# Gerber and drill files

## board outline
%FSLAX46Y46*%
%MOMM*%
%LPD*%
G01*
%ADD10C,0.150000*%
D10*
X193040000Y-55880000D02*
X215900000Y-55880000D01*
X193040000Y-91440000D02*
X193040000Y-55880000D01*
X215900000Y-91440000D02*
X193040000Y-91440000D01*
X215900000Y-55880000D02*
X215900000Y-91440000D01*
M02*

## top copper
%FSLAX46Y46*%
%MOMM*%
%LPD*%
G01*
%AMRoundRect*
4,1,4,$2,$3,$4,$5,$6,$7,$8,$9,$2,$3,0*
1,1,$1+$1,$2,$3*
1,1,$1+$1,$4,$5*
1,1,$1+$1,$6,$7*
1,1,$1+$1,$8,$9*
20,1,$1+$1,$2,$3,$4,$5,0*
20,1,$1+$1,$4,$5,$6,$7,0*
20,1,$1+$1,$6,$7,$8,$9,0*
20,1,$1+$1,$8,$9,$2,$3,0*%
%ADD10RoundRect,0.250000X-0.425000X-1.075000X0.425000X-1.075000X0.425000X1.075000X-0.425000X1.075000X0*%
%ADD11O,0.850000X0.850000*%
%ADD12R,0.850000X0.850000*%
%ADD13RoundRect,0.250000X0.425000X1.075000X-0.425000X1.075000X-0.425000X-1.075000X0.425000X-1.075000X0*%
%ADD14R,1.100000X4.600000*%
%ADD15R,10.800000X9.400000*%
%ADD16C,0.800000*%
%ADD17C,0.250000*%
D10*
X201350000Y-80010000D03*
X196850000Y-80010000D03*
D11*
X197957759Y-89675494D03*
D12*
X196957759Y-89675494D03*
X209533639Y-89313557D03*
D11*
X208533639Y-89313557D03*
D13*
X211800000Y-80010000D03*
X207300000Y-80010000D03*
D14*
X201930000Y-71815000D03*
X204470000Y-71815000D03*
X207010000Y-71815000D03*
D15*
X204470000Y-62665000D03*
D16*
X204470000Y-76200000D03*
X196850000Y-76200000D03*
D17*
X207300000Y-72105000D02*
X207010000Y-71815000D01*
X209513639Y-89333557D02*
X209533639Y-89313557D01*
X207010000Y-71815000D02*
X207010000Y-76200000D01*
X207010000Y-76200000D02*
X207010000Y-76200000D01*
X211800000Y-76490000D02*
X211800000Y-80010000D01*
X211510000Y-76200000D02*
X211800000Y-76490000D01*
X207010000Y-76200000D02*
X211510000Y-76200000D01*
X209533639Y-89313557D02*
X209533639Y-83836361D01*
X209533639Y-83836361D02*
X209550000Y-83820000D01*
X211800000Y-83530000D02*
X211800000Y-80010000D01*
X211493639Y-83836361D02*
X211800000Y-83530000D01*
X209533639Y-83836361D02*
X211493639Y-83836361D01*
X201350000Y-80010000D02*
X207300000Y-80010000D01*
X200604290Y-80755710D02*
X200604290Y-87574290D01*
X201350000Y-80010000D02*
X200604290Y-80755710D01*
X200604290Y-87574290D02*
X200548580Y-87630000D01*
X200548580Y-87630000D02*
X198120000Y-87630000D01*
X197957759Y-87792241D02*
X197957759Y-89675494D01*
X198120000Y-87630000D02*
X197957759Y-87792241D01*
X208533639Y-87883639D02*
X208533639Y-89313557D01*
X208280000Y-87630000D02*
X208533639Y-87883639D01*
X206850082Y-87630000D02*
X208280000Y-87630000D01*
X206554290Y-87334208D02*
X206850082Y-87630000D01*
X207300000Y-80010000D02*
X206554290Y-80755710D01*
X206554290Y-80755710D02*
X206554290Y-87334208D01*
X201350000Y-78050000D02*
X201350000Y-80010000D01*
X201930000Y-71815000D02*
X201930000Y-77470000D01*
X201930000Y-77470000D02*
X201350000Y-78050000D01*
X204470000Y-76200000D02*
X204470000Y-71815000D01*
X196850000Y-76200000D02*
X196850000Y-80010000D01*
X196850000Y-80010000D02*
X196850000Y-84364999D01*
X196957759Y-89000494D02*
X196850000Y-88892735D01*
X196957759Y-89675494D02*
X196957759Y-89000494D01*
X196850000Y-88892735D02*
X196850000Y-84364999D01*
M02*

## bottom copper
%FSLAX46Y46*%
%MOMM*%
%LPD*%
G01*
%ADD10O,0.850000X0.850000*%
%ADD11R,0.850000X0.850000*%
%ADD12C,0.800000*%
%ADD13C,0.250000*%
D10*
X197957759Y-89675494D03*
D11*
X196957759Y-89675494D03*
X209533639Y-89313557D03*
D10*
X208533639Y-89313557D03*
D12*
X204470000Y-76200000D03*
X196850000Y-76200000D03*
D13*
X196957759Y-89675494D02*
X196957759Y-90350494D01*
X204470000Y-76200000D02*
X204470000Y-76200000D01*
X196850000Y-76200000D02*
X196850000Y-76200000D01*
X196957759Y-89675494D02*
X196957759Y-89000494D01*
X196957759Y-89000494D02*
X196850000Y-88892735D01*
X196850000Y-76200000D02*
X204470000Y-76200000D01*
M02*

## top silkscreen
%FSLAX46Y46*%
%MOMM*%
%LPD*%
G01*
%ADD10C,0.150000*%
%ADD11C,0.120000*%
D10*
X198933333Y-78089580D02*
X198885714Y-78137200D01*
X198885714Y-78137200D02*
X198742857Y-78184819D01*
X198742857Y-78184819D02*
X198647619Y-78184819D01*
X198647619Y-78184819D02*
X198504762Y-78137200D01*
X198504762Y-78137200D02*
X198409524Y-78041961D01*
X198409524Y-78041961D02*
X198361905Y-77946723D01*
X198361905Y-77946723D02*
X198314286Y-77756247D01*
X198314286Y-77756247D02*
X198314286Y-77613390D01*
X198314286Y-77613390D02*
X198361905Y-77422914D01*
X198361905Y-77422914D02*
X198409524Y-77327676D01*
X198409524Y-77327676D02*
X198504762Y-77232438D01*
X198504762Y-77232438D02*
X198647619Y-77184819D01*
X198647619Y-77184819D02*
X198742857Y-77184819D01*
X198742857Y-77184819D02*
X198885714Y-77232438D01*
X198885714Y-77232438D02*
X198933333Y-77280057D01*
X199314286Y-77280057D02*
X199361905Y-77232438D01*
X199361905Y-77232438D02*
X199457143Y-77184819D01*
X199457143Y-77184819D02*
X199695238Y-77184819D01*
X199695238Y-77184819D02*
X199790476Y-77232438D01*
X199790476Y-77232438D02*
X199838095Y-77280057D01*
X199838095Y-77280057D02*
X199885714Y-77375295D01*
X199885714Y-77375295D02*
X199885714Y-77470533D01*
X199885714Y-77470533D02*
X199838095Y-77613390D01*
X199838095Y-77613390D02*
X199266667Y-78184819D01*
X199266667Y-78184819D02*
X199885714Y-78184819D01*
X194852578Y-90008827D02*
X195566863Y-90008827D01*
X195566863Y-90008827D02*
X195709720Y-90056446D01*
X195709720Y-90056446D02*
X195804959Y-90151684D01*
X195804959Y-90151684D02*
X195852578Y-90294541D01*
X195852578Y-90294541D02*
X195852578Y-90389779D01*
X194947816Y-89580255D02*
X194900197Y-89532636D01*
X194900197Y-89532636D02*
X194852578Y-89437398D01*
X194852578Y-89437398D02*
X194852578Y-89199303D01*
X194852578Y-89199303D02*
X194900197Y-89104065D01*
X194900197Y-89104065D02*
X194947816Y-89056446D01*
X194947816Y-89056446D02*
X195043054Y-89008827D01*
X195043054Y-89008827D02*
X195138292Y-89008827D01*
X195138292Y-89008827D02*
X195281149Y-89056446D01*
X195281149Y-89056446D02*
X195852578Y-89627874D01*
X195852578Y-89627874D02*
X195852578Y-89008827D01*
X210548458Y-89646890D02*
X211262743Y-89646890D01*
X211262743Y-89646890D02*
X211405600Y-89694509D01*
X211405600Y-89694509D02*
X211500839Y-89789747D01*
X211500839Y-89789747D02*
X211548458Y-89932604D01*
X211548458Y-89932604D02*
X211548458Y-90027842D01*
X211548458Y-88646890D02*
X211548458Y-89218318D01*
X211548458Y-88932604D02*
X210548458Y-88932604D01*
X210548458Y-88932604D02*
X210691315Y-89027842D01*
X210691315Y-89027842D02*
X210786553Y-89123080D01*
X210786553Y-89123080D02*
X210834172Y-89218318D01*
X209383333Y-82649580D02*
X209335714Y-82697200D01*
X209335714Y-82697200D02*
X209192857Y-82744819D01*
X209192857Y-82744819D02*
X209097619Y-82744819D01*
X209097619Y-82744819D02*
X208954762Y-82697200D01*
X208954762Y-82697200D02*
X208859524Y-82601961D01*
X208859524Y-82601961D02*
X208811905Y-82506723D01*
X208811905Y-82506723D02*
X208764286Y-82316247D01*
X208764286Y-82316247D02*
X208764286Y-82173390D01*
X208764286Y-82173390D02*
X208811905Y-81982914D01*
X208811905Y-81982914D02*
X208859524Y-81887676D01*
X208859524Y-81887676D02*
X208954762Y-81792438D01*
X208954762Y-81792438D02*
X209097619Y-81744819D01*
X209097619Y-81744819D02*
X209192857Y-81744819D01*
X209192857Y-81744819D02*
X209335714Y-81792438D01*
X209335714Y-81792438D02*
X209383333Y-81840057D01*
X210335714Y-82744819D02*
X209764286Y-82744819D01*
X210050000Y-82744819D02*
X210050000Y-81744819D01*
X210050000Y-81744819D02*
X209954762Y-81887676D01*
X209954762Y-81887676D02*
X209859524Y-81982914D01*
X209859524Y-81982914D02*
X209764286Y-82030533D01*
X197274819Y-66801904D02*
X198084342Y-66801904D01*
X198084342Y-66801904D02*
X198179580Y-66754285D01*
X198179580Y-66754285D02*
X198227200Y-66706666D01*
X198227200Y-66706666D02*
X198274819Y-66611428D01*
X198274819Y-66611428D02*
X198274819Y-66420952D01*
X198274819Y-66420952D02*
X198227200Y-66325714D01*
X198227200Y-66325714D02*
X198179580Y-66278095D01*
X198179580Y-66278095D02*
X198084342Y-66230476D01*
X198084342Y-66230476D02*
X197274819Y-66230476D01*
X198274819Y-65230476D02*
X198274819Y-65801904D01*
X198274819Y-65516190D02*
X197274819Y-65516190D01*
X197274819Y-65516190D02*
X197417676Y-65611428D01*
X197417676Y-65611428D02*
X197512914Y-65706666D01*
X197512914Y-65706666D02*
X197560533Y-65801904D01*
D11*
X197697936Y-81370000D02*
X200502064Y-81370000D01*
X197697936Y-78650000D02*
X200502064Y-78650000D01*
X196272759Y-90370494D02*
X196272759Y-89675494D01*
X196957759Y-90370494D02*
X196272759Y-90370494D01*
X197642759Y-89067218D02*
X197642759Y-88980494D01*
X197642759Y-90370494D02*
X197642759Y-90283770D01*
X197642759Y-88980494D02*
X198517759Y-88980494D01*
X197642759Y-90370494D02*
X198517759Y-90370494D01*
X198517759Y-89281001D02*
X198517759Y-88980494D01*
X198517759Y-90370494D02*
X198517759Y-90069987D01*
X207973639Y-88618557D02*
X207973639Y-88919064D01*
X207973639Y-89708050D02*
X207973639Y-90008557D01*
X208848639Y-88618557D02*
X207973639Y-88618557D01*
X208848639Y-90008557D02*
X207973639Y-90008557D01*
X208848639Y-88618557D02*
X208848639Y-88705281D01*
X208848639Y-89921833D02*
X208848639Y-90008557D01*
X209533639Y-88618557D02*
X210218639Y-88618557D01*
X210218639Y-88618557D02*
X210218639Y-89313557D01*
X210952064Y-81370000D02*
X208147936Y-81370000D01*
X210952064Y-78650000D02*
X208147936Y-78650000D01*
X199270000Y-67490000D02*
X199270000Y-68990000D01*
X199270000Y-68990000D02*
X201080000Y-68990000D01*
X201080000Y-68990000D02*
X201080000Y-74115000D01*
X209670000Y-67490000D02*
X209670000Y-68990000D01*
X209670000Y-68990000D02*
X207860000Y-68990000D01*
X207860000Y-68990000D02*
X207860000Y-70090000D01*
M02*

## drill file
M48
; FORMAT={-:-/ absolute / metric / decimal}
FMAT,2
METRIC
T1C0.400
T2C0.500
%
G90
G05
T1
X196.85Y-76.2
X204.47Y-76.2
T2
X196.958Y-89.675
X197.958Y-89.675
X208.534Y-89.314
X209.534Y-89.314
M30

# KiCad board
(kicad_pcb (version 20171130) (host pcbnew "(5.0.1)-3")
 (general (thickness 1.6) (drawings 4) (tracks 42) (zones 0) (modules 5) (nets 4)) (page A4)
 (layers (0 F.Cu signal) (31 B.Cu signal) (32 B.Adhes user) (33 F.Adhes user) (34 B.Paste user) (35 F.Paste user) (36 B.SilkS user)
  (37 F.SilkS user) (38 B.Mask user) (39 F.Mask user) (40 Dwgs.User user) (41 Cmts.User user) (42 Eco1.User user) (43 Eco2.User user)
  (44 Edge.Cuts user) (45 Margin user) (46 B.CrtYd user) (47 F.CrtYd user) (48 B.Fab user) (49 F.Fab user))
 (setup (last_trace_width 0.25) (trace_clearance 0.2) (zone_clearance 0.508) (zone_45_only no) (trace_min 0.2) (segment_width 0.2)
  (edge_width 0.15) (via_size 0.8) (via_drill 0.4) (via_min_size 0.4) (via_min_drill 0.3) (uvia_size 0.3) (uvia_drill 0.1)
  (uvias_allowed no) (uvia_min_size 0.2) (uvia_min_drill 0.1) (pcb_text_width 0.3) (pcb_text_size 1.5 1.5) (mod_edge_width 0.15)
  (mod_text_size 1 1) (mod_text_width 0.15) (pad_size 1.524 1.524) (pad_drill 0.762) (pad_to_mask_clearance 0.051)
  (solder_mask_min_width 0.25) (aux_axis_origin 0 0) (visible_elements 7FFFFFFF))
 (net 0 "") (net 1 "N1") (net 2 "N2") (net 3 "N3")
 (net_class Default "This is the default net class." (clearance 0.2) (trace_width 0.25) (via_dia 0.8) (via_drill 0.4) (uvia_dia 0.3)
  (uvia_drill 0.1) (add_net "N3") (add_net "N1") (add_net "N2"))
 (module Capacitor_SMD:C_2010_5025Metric (layer F.Cu) (at 199.1 80.01)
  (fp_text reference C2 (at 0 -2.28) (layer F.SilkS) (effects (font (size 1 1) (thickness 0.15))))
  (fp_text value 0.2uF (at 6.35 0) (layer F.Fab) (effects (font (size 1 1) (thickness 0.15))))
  (fp_line (start -1.402064 1.36) (end 1.402064 1.36) (layer F.SilkS) (width 0.12))
  (fp_line (start -1.402064 -1.36) (end 1.402064 -1.36) (layer F.SilkS) (width 0.12))
  (pad 2 smd roundrect (at 2.25 0) (size 1.35 2.65) (layers F.Cu F.Paste F.Mask) (roundrect_rratio 0.185185) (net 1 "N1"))
  (pad 1 smd roundrect (at -2.25 0) (size 1.35 2.65) (layers F.Cu F.Paste F.Mask) (roundrect_rratio 0.185185) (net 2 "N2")))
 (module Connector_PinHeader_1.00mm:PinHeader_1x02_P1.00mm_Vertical (layer F.Cu) (at 196.957759 89.675494 90)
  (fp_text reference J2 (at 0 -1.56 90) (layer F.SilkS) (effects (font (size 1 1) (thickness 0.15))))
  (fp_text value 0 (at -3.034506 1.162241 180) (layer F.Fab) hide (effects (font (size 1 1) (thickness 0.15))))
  (fp_line (start -0.695 -0.685) (end 0 -0.685) (layer F.SilkS) (width 0.12))
  (fp_line (start -0.695 0) (end -0.695 -0.685) (layer F.SilkS) (width 0.12))
  (fp_line (start 0.608276 0.685) (end 0.695 0.685) (layer F.SilkS) (width 0.12))
  (fp_line (start -0.695 0.685) (end -0.608276 0.685) (layer F.SilkS) (width 0.12))
  (fp_line (start 0.695 0.685) (end 0.695 1.56) (layer F.SilkS) (width 0.12))
  (fp_line (start -0.695 0.685) (end -0.695 1.56) (layer F.SilkS) (width 0.12))
  (fp_line (start 0.394493 1.56) (end 0.695 1.56) (layer F.SilkS) (width 0.12))
  (fp_line (start -0.695 1.56) (end -0.394493 1.56) (layer F.SilkS) (width 0.12))
  (pad 2 thru_hole oval (at 0 1 90) (size 0.85 0.85) (drill 0.5) (layers *.Cu *.Mask) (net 1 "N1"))
  (pad 1 thru_hole rect (at 0 0 90) (size 0.85 0.85) (drill 0.5) (layers *.Cu *.Mask) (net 2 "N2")))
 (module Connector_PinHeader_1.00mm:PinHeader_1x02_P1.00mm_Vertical (layer F.Cu) (at 209.533639 89.313557 270)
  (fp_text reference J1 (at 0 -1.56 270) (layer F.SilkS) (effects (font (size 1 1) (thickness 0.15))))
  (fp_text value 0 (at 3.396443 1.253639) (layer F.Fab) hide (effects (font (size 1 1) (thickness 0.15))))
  (fp_line (start -0.695 1.56) (end -0.394493 1.56) (layer F.SilkS) (width 0.12))
  (fp_line (start 0.394493 1.56) (end 0.695 1.56) (layer F.SilkS) (width 0.12))
  (fp_line (start -0.695 0.685) (end -0.695 1.56) (layer F.SilkS) (width 0.12))
  (fp_line (start 0.695 0.685) (end 0.695 1.56) (layer F.SilkS) (width 0.12))
  (fp_line (start -0.695 0.685) (end -0.608276 0.685) (layer F.SilkS) (width 0.12))
  (fp_line (start 0.608276 0.685) (end 0.695 0.685) (layer F.SilkS) (width 0.12))
  (fp_line (start -0.695 0) (end -0.695 -0.685) (layer F.SilkS) (width 0.12))
  (fp_line (start -0.695 -0.685) (end 0 -0.685) (layer F.SilkS) (width 0.12))
  (pad 1 thru_hole rect (at 0 0 270) (size 0.85 0.85) (drill 0.5) (layers *.Cu *.Mask) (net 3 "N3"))
  (pad 2 thru_hole oval (at 0 1 270) (size 0.85 0.85) (drill 0.5) (layers *.Cu *.Mask) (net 1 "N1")))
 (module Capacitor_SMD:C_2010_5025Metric (layer F.Cu) (at 209.55 80.01 180)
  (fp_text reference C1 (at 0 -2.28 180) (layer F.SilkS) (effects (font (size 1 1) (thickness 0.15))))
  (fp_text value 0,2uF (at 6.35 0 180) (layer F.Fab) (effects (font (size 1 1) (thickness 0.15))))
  (fp_line (start -1.402064 -1.36) (end 1.402064 -1.36) (layer F.SilkS) (width 0.12))
  (fp_line (start -1.402064 1.36) (end 1.402064 1.36) (layer F.SilkS) (width 0.12))
  (pad 1 smd roundrect (at -2.25 0 180) (size 1.35 2.65) (layers F.Cu F.Paste F.Mask) (roundrect_rratio 0.185185) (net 3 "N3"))
  (pad 2 smd roundrect (at 2.25 0 180) (size 1.35 2.65) (layers F.Cu F.Paste F.Mask) (roundrect_rratio 0.185185) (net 1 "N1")))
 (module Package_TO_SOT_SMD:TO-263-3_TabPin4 (layer F.Cu) (at 204.47 66.04 90)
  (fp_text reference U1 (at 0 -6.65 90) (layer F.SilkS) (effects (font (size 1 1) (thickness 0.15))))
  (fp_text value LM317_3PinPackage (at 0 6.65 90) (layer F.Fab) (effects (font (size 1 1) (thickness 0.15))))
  (fp_line (start -1.45 -5.2) (end -2.95 -5.2) (layer F.SilkS) (width 0.12))
  (fp_line (start -2.95 -5.2) (end -2.95 -3.39) (layer F.SilkS) (width 0.12))
  (fp_line (start -2.95 -3.39) (end -8.075 -3.39) (layer F.SilkS) (width 0.12))
  (fp_line (start -1.45 5.2) (end -2.95 5.2) (layer F.SilkS) (width 0.12))
  (fp_line (start -2.95 5.2) (end -2.95 3.39) (layer F.SilkS) (width 0.12))
  (fp_line (start -2.95 3.39) (end -4.05 3.39) (layer F.SilkS) (width 0.12))
  (pad 1 smd rect (at -5.775 -2.54 90) (size 4.6 1.1) (layers F.Cu F.Paste F.Mask) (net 1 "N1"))
  (pad 2 smd rect (at -5.775 0 90) (size 4.6 1.1) (layers F.Cu F.Paste F.Mask) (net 2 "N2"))
  (pad 3 smd rect (at -5.775 2.54 90) (size 4.6 1.1) (layers F.Cu F.Paste F.Mask) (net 3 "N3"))
  (pad 4 smd rect (at 3.375 0 90) (size 9.4 10.8) (layers F.Cu F.Mask))
  (pad "" smd rect (at 5.8 2.775 90) (size 4.55 5.25) (layers F.Paste))
  (pad "" smd rect (at 0.95 -2.775 90) (size 4.55 5.25) (layers F.Paste))
  (pad "" smd rect (at 5.8 -2.775 90) (size 4.55 5.25) (layers F.Paste))
  (pad "" smd rect (at 0.95 2.775 90) (size 4.55 5.25) (layers F.Paste)))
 (gr_line (start 193.04 55.88) (end 215.9 55.88) (layer Edge.Cuts) (width 0.15))
 (gr_line (start 193.04 91.44) (end 193.04 55.88) (layer Edge.Cuts) (width 0.15))
 (gr_line (start 215.9 91.44) (end 193.04 91.44) (layer Edge.Cuts) (width 0.15))
 (gr_line (start 215.9 55.88) (end 215.9 91.44) (layer Edge.Cuts) (width 0.15))
 (segment (start 207.3 72.105) (end 207.01 71.815) (width 0.25) (layer F.Cu) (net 3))
 (segment (start 209.513639 89.333557) (end 209.533639 89.313557) (width 0.25) (layer F.Cu) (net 3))
 (segment (start 207.01 71.815) (end 207.01 76.2) (width 0.25) (layer F.Cu) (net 3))
 (segment (start 207.01 76.2) (end 207.01 76.2) (width 0.25) (layer F.Cu) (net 3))
 (segment (start 211.8 76.49) (end 211.8 80.01) (width 0.25) (layer F.Cu) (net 3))
 (segment (start 211.51 76.2) (end 211.8 76.49) (width 0.25) (layer F.Cu) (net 3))
 (segment (start 207.01 76.2) (end 211.51 76.2) (width 0.25) (layer F.Cu) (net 3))
 (segment (start 209.533639 89.313557) (end 209.533639 83.836361) (width 0.25) (layer F.Cu) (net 3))
 (segment (start 209.533639 83.836361) (end 209.55 83.82) (width 0.25) (layer F.Cu) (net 3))
 (segment (start 211.8 83.53) (end 211.8 80.01) (width 0.25) (layer F.Cu) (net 3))
 (segment (start 211.493639 83.836361) (end 211.8 83.53) (width 0.25) (layer F.Cu) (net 3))
 (segment (start 209.533639 83.836361) (end 211.493639 83.836361) (width 0.25) (layer F.Cu) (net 3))
 (segment (start 201.35 80.01) (end 207.3 80.01) (width 0.25) (layer F.Cu) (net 1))
 (segment (start 200.60429 80.75571) (end 200.60429 87.57429) (width 0.25) (layer F.Cu) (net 1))
 (segment (start 201.35 80.01) (end 200.60429 80.75571) (width 0.25) (layer F.Cu) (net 1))
 (segment (start 200.60429 87.57429) (end 200.54858 87.63) (width 0.25) (layer F.Cu) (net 1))
 (segment (start 200.54858 87.63) (end 198.12 87.63) (width 0.25) (layer F.Cu) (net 1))
 (segment (start 197.957759 87.792241) (end 197.957759 89.675494) (width 0.25) (layer F.Cu) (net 1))
 (segment (start 198.12 87.63) (end 197.957759 87.792241) (width 0.25) (layer F.Cu) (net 1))
 (segment (start 208.533639 87.883639) (end 208.533639 89.313557) (width 0.25) (layer F.Cu) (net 1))
 (segment (start 208.28 87.63) (end 208.533639 87.883639) (width 0.25) (layer F.Cu) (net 1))
 (segment (start 206.850082 87.63) (end 208.28 87.63) (width 0.25) (layer F.Cu) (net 1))
 (segment (start 206.55429 87.334208) (end 206.850082 87.63) (width 0.25) (layer F.Cu) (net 1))
 (segment (start 207.3 80.01) (end 206.55429 80.75571) (width 0.25) (layer F.Cu) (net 1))
 (segment (start 206.55429 80.75571) (end 206.55429 87.334208) (width 0.25) (layer F.Cu) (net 1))
 (segment (start 201.35 78.05) (end 201.35 80.01) (width 0.25) (layer F.Cu) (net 1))
 (segment (start 201.93 71.815) (end 201.93 77.47) (width 0.25) (layer F.Cu) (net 1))
 (segment (start 201.93 77.47) (end 201.35 78.05) (width 0.25) (layer F.Cu) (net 1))
 (segment (start 196.957759 89.675494) (end 196.957759 90.350494) (width 0.25) (layer B.Cu) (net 2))
 (segment (start 204.47 76.2) (end 204.47 76.2) (width 0.25) (layer B.Cu) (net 2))
 (via (at 204.47 76.2) (size 0.8) (drill 0.4) (layers F.Cu B.Cu) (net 2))
 (segment (start 204.47 76.2) (end 204.47 71.815) (width 0.25) (layer F.Cu) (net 2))
 (segment (start 196.85 76.2) (end 196.85 76.2) (width 0.25) (layer B.Cu) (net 2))
 (segment (start 196.957759 89.675494) (end 196.957759 89.000494) (width 0.25) (layer B.Cu) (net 2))
 (segment (start 196.957759 89.000494) (end 196.85 88.892735) (width 0.25) (layer B.Cu) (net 2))
 (segment (start 196.85 76.2) (end 204.47 76.2) (width 0.25) (layer B.Cu) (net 2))
 (via (at 196.85 76.2) (size 0.8) (drill 0.4) (layers F.Cu B.Cu) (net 2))
 (segment (start 196.85 76.2) (end 196.85 80.01) (width 0.25) (layer F.Cu) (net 2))
 (segment (start 196.85 80.01) (end 196.85 84.364999) (width 0.25) (layer F.Cu) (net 2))
 (segment (start 196.957759 89.000494) (end 196.85 88.892735) (width 0.25) (layer F.Cu) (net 2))
 (segment (start 196.957759 89.675494) (end 196.957759 89.000494) (width 0.25) (layer F.Cu) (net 2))
 (segment (start 196.85 88.892735) (end 196.85 84.364999) (width 0.25) (layer F.Cu) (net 2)))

